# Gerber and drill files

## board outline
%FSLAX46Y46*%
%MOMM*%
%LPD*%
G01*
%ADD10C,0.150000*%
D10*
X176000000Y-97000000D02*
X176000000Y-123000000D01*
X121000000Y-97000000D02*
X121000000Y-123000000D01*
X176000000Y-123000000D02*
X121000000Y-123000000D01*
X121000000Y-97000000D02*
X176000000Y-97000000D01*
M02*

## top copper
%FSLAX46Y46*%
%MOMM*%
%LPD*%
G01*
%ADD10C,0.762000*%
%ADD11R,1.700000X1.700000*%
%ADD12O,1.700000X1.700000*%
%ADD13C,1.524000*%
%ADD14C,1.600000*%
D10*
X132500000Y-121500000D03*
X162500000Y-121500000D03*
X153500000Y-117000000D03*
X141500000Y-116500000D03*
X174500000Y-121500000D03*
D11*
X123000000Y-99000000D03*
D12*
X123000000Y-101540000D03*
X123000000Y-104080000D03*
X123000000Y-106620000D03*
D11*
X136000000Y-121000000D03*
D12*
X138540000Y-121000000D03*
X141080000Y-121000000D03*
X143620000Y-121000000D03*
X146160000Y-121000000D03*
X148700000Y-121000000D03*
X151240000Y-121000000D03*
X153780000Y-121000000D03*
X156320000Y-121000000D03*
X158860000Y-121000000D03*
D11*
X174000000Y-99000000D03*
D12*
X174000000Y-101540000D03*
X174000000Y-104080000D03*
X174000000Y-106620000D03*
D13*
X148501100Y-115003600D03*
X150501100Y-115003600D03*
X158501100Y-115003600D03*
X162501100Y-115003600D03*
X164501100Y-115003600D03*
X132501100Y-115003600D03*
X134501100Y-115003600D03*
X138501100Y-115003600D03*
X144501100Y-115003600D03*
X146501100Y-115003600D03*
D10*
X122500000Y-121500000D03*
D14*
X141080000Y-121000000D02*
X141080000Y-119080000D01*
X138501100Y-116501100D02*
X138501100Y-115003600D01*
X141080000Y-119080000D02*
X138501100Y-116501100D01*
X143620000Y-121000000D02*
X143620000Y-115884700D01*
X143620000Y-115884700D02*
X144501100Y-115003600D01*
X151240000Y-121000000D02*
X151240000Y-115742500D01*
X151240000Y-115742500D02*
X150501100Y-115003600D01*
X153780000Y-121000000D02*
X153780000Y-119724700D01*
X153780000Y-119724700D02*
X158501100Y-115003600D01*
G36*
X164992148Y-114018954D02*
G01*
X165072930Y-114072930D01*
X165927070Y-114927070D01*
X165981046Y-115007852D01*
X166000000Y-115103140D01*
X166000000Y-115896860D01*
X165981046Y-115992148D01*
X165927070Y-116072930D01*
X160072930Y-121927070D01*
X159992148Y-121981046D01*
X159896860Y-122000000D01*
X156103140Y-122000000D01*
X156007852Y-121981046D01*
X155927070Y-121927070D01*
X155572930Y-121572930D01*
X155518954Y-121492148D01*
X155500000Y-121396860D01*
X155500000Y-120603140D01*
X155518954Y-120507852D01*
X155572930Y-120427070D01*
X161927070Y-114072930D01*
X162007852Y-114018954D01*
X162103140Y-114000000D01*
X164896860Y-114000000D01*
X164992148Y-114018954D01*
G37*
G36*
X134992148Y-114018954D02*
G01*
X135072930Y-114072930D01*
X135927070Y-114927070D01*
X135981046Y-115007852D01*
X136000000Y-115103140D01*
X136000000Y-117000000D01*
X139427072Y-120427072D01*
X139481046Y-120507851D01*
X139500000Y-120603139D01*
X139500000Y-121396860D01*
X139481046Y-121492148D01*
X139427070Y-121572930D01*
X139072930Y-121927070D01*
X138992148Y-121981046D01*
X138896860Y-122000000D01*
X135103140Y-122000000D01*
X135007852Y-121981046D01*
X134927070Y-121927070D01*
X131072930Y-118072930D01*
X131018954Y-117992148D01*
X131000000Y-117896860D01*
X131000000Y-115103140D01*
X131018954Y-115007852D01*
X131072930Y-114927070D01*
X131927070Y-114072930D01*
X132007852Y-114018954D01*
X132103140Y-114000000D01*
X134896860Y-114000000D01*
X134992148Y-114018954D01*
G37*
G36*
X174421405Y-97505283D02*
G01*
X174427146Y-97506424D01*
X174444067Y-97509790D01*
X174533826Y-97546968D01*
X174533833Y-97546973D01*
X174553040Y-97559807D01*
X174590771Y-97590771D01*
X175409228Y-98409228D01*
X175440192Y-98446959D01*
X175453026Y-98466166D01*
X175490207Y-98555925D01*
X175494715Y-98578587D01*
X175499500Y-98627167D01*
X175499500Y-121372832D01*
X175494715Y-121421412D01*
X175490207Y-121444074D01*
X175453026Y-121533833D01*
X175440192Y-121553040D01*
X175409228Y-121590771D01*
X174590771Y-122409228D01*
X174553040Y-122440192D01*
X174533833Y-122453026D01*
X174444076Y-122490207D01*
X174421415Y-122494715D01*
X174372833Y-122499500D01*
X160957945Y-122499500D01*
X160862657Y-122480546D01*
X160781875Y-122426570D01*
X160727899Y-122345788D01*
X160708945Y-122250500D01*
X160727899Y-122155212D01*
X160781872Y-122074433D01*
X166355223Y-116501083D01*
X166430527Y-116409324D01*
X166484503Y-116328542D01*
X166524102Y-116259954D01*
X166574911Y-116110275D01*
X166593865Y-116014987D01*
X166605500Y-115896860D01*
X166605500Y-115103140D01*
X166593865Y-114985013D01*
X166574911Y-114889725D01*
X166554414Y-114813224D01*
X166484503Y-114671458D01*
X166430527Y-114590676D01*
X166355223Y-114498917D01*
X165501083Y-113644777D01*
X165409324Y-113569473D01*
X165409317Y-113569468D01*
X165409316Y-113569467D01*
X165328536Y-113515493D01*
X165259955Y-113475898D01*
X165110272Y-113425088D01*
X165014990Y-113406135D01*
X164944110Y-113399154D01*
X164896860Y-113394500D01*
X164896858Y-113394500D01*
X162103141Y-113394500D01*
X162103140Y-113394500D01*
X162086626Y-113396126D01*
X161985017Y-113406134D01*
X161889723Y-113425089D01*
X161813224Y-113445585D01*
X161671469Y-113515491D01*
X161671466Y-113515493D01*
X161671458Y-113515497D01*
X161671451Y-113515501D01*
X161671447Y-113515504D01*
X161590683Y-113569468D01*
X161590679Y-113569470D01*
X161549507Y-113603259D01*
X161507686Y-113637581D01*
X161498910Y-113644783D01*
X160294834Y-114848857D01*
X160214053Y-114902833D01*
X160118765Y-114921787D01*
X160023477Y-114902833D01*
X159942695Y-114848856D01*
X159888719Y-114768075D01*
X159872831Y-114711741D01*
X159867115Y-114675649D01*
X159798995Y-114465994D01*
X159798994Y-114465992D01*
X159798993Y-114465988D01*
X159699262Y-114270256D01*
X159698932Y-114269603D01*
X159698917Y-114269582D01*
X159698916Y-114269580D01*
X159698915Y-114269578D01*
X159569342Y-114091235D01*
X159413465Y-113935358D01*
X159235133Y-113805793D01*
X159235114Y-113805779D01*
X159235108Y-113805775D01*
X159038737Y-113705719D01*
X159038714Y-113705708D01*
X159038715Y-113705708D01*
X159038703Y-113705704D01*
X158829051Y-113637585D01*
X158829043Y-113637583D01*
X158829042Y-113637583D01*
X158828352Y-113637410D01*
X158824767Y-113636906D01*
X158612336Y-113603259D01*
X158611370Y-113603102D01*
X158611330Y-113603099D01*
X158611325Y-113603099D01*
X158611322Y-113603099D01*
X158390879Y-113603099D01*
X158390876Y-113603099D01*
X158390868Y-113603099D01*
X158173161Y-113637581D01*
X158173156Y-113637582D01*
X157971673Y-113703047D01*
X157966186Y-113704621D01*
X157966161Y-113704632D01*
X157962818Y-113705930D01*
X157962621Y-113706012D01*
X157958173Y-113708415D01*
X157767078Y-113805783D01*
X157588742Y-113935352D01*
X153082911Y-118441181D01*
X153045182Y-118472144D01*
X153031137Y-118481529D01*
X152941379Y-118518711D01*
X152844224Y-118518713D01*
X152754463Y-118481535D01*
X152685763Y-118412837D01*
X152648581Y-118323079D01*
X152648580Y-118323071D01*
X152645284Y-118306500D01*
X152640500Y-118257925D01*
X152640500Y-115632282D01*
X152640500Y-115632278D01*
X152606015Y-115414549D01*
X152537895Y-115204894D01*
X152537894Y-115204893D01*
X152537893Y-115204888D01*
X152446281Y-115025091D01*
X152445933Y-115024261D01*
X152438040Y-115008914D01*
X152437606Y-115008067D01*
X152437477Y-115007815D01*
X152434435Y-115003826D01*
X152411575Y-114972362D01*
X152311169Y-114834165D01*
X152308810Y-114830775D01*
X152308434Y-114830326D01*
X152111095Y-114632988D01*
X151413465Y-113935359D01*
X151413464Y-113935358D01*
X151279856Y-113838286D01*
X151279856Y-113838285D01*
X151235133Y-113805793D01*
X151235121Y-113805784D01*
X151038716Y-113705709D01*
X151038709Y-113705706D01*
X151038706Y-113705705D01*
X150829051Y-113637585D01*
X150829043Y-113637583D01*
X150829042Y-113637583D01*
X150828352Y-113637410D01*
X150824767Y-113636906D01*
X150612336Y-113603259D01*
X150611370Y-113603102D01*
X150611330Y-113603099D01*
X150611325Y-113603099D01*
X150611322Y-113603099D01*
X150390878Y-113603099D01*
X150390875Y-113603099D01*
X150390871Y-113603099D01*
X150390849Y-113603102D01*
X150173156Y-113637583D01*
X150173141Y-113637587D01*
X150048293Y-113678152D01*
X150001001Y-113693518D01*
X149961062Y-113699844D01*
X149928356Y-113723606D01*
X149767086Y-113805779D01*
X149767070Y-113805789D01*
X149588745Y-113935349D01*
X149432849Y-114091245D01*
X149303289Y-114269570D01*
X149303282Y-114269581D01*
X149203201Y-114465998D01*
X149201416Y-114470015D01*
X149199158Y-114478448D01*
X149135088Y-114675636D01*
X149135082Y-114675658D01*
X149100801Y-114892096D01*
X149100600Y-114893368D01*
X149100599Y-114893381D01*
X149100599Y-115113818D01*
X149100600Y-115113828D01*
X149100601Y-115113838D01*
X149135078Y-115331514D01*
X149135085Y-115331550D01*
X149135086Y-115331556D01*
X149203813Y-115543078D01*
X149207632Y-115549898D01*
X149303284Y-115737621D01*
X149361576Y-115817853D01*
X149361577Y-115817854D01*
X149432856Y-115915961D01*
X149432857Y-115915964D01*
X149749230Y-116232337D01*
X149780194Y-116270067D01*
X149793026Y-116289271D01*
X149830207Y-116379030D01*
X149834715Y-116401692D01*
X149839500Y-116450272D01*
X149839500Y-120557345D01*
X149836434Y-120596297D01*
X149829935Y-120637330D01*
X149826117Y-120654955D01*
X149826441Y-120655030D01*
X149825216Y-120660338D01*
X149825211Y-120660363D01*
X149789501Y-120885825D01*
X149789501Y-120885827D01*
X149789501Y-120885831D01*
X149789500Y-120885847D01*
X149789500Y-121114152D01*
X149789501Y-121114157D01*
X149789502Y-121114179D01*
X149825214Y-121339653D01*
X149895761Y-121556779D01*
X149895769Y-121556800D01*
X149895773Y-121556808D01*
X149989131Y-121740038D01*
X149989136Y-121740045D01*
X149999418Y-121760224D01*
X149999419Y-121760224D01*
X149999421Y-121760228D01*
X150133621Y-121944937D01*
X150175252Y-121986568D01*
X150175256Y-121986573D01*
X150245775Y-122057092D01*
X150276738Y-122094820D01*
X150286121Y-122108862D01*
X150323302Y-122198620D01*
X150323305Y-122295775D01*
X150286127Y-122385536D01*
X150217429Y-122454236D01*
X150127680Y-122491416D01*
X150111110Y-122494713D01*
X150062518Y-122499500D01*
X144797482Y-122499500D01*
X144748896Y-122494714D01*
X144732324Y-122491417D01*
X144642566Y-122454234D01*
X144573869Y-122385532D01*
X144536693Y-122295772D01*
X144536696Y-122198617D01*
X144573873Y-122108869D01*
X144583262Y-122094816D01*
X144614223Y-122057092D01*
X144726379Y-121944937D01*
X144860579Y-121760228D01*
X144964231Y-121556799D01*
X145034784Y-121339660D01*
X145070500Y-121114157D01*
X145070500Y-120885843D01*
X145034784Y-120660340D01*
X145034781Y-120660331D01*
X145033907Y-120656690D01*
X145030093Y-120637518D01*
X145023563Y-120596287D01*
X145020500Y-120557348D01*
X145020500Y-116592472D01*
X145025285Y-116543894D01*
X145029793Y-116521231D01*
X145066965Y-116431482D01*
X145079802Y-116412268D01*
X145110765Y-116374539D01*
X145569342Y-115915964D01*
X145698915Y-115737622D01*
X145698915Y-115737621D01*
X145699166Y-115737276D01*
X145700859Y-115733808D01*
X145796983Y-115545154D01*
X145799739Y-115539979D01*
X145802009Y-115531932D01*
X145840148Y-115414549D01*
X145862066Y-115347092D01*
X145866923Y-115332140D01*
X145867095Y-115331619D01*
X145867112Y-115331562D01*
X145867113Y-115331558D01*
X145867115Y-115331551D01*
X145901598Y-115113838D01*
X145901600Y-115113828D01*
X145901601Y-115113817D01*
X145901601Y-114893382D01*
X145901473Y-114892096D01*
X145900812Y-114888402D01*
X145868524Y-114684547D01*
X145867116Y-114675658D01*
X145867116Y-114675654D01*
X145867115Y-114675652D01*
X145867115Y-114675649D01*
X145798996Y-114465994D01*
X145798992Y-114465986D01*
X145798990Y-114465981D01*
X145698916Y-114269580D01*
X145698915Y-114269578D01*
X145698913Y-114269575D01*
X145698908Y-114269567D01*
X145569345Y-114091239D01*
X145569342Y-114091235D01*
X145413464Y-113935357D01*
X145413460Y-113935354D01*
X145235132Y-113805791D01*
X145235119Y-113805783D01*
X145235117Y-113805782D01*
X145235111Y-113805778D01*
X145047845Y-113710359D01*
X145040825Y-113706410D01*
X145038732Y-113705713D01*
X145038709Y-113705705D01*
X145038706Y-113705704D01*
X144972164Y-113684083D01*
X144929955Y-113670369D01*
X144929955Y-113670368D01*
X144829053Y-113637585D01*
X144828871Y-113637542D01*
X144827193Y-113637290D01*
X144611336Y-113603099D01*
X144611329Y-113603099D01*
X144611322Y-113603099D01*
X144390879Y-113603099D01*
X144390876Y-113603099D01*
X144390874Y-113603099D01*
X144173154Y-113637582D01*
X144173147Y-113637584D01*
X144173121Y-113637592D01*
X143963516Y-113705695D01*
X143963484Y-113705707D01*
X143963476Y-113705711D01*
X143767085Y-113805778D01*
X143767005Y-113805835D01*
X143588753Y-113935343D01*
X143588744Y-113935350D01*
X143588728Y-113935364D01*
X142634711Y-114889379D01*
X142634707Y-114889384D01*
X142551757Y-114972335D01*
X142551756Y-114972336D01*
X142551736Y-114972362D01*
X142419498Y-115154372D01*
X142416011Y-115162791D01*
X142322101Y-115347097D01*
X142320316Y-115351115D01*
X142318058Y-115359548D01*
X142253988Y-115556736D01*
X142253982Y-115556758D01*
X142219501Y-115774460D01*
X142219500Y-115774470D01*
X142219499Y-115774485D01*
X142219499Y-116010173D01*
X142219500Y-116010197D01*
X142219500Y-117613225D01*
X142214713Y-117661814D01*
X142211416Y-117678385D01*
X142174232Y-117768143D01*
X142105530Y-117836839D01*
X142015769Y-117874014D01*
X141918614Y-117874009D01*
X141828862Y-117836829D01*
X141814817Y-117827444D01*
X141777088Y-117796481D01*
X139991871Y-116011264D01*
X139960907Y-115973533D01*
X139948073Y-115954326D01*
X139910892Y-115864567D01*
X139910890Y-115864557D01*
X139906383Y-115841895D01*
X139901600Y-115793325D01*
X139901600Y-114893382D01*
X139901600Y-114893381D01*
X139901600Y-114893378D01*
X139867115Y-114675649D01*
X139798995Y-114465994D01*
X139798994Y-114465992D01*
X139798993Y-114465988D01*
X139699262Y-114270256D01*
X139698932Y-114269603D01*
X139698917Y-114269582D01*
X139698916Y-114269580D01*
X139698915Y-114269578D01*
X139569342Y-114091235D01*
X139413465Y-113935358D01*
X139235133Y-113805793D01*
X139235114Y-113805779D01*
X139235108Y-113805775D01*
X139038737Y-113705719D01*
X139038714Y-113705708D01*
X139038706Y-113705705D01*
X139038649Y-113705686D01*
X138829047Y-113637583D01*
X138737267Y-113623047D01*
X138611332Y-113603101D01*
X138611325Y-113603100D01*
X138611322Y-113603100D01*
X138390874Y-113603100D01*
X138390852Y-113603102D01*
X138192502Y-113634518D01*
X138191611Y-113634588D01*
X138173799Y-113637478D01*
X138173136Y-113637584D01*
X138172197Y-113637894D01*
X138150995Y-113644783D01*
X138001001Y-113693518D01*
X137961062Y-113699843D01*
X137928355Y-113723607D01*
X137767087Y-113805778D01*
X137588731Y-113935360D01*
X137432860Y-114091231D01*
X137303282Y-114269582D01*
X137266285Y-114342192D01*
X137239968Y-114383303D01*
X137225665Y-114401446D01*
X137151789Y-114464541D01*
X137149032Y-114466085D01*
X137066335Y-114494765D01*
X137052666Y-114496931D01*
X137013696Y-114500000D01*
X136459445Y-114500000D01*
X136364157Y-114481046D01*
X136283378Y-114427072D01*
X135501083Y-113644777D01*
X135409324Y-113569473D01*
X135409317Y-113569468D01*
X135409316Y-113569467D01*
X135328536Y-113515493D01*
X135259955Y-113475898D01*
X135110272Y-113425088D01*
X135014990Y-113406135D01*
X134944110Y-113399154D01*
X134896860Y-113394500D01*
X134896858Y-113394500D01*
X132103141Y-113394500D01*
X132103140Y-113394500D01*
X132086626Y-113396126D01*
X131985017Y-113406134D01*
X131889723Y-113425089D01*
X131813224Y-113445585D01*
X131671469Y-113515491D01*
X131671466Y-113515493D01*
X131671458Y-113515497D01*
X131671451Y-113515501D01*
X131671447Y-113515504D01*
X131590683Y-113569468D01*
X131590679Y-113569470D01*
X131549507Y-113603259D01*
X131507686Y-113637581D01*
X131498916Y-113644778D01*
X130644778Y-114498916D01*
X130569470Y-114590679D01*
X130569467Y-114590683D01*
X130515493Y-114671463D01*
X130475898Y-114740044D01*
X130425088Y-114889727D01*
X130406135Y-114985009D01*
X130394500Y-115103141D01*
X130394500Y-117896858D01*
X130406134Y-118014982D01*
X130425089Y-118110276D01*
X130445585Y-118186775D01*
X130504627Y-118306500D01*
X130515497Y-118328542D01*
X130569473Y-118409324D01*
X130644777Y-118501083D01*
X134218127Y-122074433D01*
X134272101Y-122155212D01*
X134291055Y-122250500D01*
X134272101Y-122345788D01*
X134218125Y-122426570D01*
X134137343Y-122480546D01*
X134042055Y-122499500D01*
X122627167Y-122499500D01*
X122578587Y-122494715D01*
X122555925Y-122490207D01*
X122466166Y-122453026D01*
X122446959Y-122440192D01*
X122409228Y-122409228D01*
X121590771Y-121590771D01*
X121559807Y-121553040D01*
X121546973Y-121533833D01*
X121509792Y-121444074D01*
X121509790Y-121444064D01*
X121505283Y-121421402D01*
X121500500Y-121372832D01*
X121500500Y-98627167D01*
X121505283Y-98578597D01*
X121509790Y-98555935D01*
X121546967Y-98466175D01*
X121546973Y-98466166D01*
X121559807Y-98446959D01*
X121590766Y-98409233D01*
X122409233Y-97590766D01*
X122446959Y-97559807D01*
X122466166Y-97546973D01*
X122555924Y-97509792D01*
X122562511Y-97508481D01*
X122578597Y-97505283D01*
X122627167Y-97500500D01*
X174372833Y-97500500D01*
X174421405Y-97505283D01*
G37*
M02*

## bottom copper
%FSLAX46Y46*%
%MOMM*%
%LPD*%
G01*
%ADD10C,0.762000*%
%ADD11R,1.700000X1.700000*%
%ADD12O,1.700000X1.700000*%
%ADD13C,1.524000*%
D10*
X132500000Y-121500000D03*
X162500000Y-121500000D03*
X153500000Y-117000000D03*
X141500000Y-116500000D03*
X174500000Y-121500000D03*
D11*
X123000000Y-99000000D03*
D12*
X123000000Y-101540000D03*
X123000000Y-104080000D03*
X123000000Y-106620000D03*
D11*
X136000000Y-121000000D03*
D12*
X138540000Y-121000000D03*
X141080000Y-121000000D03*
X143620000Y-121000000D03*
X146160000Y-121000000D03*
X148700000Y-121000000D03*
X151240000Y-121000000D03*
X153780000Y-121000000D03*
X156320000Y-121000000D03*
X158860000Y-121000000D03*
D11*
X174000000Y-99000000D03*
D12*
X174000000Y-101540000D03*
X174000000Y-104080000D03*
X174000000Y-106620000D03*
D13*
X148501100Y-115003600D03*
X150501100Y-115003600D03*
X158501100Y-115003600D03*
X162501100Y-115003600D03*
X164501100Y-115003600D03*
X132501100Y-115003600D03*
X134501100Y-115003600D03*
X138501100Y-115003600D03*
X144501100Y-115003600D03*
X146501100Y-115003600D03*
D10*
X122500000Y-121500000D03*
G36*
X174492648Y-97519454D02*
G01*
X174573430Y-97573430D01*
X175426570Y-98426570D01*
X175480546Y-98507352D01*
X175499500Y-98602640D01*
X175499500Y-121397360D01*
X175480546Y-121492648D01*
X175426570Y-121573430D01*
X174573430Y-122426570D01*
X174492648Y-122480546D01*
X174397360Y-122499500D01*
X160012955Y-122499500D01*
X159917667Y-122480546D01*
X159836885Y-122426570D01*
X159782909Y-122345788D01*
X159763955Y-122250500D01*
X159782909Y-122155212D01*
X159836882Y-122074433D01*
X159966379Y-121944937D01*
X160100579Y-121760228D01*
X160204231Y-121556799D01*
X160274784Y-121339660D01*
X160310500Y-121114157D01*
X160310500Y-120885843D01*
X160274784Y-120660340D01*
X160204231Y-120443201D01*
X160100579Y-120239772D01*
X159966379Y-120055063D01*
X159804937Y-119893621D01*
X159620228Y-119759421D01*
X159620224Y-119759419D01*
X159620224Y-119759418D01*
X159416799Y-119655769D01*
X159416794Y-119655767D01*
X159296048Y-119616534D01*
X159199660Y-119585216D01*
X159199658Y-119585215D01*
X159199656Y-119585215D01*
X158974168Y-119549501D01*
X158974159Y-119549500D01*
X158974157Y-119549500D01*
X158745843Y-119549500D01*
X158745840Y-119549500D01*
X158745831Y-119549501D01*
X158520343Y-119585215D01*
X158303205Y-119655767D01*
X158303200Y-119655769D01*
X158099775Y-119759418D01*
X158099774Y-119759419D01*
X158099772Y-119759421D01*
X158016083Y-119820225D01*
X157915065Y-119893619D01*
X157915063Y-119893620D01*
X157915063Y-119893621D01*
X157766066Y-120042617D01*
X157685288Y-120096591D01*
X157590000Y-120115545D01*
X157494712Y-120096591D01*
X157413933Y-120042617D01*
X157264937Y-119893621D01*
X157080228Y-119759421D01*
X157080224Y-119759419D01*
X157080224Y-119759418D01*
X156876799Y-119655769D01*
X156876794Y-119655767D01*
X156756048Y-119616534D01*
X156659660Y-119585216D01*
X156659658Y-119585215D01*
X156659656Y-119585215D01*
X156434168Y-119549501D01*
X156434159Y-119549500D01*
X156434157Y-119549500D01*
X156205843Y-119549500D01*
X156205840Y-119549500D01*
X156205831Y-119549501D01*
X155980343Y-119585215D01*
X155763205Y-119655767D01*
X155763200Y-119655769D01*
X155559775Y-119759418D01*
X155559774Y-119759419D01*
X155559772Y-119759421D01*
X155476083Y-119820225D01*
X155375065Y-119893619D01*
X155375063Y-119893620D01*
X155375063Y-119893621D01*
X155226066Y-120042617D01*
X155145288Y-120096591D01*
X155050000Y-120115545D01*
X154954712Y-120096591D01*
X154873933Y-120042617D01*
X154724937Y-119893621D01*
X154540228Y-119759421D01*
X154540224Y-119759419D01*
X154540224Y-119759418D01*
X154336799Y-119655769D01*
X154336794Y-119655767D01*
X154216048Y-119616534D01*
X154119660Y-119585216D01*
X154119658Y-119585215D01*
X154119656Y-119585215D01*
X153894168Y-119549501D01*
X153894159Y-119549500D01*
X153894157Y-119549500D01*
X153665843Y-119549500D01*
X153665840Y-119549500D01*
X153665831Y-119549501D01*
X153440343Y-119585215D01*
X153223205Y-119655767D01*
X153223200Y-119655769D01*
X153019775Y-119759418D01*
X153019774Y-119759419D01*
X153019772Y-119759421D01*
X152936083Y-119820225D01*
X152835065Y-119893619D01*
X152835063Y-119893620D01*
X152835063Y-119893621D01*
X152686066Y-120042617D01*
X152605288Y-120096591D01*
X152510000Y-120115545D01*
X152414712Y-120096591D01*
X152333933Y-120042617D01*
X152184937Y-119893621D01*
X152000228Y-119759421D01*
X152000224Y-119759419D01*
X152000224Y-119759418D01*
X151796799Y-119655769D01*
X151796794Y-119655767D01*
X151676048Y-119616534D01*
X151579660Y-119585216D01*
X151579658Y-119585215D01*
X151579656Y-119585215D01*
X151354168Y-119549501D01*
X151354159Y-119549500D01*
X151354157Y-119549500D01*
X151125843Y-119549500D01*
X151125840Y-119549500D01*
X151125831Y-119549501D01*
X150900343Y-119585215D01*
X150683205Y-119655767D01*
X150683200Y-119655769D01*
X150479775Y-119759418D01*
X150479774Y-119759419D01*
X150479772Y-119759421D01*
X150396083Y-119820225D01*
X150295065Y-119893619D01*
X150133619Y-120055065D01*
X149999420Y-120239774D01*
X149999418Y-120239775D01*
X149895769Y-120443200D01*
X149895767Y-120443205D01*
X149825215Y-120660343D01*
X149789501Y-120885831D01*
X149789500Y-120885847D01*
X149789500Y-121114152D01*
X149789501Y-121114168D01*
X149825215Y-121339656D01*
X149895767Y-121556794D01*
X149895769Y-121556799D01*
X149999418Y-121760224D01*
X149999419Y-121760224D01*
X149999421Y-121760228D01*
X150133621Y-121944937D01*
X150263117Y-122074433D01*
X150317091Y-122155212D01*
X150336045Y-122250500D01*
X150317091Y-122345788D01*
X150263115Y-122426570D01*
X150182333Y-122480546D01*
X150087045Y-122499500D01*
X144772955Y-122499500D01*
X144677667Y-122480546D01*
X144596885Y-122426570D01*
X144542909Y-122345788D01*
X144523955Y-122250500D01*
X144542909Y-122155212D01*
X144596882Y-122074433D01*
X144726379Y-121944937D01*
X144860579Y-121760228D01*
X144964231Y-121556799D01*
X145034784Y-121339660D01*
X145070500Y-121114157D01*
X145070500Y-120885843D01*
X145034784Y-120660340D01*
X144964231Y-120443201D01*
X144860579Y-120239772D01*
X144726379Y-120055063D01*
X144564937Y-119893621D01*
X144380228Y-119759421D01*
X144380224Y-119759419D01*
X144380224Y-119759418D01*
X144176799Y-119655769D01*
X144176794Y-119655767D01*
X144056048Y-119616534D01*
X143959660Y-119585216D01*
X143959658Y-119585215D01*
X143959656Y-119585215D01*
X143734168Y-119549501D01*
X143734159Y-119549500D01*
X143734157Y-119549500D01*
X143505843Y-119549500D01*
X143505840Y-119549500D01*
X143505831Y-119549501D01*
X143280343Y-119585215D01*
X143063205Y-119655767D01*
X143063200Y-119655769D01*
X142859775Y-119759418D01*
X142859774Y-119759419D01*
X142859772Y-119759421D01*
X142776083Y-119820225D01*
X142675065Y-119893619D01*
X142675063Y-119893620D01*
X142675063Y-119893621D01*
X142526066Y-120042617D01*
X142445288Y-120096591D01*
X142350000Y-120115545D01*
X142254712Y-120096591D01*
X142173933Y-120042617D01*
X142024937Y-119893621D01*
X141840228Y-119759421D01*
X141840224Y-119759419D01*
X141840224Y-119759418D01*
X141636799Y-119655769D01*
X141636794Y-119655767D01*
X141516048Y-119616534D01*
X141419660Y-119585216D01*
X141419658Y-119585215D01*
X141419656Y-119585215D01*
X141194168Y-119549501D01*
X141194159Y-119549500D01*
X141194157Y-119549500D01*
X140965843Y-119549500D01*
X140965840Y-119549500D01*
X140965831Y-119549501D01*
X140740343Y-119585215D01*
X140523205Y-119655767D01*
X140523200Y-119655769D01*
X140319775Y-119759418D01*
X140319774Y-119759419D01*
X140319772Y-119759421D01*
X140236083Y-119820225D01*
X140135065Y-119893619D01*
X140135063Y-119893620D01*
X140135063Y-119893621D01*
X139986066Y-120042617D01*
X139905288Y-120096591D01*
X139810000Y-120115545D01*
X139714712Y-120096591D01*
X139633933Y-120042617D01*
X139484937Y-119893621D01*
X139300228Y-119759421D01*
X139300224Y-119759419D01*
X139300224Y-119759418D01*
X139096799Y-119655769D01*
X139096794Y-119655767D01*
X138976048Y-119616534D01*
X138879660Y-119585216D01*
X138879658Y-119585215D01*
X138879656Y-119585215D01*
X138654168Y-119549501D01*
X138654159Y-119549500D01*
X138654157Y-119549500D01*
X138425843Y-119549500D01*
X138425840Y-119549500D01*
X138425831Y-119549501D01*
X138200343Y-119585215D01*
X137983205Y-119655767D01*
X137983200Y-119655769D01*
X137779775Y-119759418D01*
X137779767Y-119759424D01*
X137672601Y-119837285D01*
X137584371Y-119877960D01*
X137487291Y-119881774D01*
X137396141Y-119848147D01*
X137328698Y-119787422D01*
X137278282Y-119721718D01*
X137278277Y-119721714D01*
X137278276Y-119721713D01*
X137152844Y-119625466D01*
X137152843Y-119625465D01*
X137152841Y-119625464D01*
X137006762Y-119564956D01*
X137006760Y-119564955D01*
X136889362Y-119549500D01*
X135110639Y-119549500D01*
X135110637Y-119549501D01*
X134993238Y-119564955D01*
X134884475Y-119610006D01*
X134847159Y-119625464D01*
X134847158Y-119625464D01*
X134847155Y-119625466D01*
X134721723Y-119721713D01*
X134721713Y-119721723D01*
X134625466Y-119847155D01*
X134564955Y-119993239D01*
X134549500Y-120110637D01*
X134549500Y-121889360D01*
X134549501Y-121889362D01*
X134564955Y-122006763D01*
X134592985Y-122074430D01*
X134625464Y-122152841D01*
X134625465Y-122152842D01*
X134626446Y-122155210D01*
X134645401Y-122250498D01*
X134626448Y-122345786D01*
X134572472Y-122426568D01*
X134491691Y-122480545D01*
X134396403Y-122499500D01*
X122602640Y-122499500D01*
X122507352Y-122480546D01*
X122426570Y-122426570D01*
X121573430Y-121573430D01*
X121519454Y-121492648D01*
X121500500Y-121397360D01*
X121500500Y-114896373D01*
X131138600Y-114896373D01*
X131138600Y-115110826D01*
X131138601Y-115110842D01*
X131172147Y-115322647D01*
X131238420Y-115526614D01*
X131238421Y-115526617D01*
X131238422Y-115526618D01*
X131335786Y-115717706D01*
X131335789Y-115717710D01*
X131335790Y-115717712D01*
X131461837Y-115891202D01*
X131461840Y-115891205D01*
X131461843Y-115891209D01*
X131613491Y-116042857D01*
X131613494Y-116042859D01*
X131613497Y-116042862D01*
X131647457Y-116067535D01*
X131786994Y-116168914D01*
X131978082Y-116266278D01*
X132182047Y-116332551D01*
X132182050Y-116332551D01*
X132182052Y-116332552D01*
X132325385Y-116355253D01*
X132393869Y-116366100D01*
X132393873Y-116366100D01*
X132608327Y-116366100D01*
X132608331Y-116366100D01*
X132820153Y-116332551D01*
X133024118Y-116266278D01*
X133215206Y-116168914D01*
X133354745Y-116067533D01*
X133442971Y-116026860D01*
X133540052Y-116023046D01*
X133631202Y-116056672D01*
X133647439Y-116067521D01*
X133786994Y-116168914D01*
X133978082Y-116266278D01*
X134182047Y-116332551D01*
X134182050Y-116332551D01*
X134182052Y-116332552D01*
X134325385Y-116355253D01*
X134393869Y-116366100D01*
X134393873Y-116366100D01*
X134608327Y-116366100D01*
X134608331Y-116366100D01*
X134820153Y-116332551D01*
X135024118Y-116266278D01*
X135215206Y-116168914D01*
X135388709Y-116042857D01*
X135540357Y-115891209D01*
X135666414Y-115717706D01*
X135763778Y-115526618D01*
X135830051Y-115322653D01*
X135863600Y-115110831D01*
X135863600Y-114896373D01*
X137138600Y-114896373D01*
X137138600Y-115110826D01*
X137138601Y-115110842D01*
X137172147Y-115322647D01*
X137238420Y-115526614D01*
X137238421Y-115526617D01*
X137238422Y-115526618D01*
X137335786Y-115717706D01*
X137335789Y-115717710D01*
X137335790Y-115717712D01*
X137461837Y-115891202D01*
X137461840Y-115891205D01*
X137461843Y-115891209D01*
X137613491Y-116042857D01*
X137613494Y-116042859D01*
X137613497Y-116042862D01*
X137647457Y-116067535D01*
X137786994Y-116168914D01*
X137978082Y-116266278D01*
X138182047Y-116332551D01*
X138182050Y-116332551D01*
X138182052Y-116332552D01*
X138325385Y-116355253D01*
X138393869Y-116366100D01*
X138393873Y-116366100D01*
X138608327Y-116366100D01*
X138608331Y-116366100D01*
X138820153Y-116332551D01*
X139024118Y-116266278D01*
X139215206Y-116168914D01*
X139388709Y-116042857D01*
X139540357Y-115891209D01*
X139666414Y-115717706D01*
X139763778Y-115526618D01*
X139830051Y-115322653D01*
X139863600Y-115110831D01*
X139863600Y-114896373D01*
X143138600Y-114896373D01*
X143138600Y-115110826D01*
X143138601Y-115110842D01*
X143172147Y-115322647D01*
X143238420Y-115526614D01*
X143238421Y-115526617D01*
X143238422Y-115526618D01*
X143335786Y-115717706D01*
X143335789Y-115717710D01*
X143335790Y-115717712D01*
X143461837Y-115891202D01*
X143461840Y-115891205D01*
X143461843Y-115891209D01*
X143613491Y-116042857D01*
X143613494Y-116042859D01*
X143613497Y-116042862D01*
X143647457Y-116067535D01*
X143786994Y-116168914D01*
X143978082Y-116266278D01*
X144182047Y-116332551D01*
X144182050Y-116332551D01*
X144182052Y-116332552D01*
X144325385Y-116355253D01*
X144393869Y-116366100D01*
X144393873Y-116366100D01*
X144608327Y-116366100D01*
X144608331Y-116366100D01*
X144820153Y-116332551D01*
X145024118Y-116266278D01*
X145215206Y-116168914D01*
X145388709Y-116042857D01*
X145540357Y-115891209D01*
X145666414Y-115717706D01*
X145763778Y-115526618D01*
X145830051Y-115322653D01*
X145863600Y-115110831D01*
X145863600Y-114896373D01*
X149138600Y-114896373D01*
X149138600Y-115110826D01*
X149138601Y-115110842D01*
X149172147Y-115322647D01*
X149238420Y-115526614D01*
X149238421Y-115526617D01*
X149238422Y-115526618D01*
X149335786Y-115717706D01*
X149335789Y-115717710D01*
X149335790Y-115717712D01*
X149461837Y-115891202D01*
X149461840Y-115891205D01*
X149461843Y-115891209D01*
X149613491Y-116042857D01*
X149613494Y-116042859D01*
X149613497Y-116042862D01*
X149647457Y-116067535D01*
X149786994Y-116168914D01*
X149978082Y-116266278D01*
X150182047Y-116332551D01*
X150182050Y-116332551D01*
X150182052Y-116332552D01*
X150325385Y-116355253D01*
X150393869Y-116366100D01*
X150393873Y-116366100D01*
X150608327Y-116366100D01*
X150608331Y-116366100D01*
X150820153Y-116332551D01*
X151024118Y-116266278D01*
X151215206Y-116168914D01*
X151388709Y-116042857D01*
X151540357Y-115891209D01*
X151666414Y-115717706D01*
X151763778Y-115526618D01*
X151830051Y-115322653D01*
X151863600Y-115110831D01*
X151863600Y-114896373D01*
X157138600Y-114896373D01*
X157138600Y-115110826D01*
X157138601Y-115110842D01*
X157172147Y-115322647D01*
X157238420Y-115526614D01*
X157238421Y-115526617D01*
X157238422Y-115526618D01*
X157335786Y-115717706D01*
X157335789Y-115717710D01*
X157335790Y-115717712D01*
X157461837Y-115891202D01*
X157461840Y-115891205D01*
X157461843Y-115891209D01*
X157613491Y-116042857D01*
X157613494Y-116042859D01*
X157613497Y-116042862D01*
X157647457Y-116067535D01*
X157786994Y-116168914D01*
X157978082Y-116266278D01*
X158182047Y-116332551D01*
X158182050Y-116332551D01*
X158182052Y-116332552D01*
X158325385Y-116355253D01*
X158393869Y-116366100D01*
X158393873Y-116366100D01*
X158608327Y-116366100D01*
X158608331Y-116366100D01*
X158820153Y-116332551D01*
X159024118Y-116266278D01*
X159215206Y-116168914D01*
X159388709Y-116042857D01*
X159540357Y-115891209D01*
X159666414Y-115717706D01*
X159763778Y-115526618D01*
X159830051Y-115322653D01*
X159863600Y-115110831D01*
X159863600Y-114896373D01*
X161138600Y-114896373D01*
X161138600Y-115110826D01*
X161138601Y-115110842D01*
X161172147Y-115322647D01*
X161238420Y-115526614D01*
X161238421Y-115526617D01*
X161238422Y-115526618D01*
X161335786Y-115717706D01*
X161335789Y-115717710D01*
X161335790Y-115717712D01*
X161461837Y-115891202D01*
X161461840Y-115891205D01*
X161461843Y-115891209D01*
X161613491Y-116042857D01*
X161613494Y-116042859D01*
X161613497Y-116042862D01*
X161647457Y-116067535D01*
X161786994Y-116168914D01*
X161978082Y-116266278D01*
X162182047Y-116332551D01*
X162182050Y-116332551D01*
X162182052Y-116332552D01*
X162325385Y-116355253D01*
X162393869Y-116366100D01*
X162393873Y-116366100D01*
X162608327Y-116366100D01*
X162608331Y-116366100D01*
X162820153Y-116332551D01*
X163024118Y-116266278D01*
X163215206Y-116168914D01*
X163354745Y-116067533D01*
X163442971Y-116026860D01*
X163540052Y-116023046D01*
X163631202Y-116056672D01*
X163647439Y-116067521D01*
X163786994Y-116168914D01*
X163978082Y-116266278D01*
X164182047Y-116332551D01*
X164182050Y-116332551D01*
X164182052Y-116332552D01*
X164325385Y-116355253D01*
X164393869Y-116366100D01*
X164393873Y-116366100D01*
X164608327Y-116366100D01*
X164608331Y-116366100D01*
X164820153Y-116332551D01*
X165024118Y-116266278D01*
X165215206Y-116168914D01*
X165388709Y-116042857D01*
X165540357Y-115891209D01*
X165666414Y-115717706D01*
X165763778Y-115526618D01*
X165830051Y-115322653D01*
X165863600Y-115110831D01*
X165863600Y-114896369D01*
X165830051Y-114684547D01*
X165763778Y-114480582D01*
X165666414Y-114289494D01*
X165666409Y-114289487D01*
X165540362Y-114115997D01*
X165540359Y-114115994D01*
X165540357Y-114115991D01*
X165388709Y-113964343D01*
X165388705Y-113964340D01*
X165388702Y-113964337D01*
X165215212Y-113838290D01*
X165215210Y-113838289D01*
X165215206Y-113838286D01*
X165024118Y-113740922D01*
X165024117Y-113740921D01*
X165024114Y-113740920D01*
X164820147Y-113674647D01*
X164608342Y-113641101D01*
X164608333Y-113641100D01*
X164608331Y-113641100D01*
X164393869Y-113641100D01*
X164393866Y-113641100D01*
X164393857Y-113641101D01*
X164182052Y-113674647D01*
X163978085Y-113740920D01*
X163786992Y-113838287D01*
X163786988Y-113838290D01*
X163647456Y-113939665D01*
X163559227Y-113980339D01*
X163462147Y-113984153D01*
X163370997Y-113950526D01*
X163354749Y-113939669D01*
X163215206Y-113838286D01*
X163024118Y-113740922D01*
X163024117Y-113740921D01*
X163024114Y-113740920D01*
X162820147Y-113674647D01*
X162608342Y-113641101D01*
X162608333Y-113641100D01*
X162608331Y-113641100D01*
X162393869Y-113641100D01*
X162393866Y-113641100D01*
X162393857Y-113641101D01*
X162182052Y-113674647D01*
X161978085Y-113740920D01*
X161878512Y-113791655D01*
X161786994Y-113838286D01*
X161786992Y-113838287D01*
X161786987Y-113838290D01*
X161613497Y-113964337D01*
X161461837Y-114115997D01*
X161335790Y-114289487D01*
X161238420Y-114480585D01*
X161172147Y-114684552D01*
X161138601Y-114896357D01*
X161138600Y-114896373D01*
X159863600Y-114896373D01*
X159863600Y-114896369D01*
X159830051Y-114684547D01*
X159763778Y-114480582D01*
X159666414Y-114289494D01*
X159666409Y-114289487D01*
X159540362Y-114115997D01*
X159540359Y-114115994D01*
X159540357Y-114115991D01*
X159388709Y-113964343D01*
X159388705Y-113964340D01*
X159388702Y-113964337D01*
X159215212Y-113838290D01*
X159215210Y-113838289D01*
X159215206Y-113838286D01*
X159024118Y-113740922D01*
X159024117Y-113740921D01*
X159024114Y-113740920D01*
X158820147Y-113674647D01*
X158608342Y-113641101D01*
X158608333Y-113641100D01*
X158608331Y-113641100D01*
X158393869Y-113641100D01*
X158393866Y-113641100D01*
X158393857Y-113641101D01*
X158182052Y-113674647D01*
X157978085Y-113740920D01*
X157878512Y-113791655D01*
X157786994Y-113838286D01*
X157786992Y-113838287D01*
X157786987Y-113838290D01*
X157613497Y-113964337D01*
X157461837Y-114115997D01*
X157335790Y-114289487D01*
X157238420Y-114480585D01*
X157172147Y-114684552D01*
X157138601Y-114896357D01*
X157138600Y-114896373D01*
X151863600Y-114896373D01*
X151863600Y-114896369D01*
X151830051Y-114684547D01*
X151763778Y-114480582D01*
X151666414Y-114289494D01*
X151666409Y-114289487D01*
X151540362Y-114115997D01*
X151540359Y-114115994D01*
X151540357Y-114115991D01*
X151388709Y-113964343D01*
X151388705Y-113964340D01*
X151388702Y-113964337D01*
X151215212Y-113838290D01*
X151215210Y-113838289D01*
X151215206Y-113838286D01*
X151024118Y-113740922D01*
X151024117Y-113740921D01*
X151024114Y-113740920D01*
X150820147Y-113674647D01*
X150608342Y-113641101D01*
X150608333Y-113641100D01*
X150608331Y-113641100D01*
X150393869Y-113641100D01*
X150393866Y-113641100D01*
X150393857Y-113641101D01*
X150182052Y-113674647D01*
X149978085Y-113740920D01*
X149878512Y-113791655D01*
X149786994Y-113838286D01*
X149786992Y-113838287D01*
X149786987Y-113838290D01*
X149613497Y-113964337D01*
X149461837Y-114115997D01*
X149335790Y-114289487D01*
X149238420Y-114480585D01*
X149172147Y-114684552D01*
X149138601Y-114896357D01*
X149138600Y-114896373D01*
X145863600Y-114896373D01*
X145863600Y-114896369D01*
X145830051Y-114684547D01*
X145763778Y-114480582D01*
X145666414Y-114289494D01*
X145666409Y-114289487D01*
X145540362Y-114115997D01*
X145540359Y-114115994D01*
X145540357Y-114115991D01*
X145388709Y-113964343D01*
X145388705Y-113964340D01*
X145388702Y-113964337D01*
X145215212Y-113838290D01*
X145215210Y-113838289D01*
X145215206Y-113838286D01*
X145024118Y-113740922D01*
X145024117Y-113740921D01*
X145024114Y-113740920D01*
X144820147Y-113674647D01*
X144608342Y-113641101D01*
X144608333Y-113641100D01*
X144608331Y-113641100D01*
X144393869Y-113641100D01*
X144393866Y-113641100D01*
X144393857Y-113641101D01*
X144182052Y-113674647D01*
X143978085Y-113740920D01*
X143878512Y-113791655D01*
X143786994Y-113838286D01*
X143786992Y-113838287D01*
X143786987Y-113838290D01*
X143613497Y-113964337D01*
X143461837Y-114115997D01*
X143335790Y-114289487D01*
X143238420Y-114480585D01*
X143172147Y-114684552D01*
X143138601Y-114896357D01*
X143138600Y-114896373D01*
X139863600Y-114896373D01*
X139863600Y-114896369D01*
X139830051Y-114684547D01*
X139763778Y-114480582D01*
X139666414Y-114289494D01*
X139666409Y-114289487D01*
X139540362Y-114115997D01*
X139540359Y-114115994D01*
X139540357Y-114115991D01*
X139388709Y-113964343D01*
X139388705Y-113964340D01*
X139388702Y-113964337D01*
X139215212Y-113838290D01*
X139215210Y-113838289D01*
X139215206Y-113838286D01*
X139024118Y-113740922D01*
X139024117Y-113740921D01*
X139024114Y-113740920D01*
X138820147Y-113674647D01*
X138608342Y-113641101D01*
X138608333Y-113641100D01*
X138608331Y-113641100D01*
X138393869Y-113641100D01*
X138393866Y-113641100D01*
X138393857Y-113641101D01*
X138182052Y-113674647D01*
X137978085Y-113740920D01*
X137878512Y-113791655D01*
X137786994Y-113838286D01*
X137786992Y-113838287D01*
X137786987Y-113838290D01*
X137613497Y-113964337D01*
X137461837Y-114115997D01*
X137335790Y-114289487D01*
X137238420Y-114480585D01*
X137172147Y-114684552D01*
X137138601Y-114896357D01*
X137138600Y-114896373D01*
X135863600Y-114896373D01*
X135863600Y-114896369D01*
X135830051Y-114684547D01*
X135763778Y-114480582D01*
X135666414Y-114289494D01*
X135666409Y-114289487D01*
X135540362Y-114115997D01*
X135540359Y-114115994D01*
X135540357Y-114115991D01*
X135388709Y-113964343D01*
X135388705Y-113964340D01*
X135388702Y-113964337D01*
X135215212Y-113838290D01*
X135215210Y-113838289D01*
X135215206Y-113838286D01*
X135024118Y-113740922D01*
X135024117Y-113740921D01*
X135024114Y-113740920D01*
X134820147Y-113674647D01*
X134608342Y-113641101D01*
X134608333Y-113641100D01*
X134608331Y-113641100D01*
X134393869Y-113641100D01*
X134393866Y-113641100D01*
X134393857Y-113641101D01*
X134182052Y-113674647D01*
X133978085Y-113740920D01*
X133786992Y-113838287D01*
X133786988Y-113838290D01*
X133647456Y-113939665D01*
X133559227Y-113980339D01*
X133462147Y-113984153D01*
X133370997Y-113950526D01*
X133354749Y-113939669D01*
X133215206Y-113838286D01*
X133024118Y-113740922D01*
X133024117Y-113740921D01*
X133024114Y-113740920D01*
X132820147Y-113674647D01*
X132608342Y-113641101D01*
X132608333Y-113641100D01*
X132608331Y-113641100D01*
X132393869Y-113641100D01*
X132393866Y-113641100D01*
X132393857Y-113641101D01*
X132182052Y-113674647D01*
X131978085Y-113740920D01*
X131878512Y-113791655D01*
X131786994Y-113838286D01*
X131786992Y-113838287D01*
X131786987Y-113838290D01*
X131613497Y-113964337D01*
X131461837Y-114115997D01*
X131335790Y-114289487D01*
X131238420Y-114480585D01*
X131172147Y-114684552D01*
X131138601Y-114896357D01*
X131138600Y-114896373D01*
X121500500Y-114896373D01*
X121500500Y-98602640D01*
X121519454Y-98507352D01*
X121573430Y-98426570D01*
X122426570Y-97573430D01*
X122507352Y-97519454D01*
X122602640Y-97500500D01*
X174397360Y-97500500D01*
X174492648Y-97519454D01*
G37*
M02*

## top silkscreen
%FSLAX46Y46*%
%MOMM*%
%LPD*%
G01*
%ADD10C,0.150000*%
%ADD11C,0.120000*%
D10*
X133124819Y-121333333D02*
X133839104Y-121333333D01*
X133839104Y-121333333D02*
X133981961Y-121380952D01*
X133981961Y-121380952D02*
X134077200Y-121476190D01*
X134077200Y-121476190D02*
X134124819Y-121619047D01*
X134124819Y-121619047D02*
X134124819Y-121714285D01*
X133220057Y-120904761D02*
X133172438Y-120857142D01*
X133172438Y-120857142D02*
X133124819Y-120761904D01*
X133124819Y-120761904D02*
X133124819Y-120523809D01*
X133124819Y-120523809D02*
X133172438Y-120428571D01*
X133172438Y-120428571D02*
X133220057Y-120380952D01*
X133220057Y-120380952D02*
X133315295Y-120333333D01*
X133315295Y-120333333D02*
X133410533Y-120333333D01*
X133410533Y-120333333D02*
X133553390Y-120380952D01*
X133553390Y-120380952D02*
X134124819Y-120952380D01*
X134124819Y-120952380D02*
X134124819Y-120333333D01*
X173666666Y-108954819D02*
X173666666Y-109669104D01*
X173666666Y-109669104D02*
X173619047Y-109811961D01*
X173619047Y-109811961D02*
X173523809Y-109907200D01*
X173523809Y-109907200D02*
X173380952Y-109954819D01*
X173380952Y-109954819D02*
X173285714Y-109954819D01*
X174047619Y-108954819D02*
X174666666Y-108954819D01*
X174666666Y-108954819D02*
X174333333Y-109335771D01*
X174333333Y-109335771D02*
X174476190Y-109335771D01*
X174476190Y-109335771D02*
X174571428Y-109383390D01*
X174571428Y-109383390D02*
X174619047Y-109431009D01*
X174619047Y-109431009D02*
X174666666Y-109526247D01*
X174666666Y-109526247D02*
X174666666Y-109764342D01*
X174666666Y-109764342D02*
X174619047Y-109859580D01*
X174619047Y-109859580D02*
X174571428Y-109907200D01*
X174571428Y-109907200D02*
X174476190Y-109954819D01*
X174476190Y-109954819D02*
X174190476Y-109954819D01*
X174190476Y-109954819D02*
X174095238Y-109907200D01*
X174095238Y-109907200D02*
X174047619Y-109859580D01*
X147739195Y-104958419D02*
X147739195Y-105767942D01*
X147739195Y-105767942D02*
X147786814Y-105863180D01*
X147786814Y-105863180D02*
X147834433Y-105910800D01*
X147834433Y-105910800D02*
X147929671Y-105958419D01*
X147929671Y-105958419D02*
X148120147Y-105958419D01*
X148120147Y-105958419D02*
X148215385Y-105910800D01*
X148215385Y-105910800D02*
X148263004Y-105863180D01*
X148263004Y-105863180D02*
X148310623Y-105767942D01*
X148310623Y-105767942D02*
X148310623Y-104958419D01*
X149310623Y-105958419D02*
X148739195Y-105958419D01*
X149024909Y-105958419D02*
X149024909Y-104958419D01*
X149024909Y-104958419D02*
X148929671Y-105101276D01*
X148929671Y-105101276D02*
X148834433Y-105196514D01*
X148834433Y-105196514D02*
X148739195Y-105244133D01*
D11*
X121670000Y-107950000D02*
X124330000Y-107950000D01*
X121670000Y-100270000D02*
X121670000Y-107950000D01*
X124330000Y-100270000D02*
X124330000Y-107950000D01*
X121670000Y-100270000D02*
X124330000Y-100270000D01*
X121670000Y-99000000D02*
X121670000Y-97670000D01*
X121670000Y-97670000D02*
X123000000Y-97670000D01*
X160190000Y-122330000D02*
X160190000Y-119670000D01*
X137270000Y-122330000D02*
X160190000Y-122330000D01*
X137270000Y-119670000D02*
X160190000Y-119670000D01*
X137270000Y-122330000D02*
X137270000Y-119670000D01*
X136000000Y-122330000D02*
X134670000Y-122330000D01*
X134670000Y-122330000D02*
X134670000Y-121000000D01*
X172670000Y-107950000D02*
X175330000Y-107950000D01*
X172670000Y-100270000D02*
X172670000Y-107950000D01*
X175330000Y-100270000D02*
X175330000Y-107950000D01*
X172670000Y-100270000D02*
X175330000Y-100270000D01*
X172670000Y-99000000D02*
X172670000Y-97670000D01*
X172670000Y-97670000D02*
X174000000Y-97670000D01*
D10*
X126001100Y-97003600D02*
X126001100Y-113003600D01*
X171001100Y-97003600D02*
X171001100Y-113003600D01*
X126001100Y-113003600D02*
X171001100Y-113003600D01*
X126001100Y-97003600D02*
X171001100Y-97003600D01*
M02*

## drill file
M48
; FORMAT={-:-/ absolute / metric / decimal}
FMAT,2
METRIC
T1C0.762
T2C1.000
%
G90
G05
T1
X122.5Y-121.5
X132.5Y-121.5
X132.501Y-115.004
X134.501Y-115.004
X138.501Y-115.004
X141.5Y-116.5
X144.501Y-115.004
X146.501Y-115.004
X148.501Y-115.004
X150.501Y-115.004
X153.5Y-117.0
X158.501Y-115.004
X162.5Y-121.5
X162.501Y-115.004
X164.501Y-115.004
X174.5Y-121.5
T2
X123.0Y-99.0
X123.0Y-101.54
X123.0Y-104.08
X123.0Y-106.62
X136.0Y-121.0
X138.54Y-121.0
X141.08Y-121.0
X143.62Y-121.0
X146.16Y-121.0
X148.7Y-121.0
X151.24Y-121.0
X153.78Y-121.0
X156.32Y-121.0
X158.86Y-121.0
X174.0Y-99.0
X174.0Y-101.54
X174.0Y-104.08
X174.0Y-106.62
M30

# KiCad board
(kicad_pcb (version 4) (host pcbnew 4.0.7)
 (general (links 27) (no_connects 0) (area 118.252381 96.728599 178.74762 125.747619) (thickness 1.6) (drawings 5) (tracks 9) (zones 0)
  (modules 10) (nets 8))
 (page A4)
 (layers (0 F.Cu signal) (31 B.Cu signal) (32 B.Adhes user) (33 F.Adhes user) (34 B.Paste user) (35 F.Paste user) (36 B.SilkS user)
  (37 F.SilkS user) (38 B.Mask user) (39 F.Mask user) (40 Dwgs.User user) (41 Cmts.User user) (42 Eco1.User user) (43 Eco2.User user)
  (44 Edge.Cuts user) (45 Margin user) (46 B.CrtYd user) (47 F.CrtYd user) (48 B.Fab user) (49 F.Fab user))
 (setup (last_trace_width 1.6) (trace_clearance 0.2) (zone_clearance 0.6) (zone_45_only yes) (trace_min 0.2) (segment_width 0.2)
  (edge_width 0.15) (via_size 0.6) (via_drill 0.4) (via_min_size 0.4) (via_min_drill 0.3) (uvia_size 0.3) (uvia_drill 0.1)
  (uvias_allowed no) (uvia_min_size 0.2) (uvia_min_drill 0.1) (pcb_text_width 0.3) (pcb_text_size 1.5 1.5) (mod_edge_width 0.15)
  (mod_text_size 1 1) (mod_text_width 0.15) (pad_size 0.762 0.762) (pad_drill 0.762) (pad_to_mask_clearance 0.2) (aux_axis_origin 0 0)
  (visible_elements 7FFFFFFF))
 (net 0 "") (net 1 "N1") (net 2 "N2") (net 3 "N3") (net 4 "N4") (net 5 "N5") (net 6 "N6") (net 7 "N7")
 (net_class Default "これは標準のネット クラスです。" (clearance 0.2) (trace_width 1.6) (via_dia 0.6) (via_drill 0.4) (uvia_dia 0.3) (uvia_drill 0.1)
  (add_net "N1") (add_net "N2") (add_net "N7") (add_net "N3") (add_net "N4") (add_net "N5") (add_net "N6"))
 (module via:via (layer F.Cu) (at 132.5 121.5)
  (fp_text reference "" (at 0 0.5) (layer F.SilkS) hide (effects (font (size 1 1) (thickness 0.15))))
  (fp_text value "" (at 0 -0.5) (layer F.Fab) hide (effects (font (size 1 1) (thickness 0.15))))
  (pad 1 thru_hole circle (at 0 0) (size 0.762 0.762) (drill 0.762) (layers *.Cu *.Mask) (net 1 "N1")))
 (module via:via (layer F.Cu) (at 162.5 121.5)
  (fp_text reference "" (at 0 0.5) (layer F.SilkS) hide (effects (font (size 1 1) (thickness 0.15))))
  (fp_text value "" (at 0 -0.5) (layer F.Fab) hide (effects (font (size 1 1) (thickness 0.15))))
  (pad 1 thru_hole circle (at 0 0) (size 0.762 0.762) (drill 0.762) (layers *.Cu *.Mask) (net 1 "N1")))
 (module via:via (layer F.Cu) (at 153.5 117)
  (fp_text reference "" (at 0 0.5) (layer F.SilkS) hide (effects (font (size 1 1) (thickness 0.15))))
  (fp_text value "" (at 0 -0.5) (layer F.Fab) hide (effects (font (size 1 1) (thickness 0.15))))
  (pad 1 thru_hole circle (at 0 0) (size 0.762 0.762) (drill 0.762) (layers *.Cu *.Mask) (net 1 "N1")))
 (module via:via (layer F.Cu) (at 141.5 116.5)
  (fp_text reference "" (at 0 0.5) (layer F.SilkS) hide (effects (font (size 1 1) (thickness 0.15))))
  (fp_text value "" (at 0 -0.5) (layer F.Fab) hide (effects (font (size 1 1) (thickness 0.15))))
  (pad 1 thru_hole circle (at 0 0) (size 0.762 0.762) (drill 0.762) (layers *.Cu *.Mask) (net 1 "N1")))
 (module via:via (layer F.Cu) (at 174.5 121.5)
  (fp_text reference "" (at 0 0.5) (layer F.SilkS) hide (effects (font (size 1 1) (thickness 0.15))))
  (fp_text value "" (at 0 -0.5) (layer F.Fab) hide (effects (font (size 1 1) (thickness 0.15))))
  (pad 1 thru_hole circle (at 0 0) (size 0.762 0.762) (drill 0.762) (layers *.Cu *.Mask) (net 1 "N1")))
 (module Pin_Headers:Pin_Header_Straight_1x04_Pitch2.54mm (layer F.Cu) (at 123 99)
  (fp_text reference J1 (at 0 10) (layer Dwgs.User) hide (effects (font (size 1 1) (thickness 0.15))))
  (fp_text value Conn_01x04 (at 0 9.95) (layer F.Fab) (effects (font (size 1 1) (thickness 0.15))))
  (fp_line (start -1.33 8.95) (end 1.33 8.95) (layer F.SilkS) (width 0.12))
  (fp_line (start -1.33 1.27) (end -1.33 8.95) (layer F.SilkS) (width 0.12))
  (fp_line (start 1.33 1.27) (end 1.33 8.95) (layer F.SilkS) (width 0.12))
  (fp_line (start -1.33 1.27) (end 1.33 1.27) (layer F.SilkS) (width 0.12))
  (fp_line (start -1.33 0) (end -1.33 -1.33) (layer F.SilkS) (width 0.12))
  (fp_line (start -1.33 -1.33) (end 0 -1.33) (layer F.SilkS) (width 0.12))
  (pad 1 thru_hole rect (at 0 0) (size 1.7 1.7) (drill 1) (layers *.Cu *.Mask) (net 1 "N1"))
  (pad 2 thru_hole oval (at 0 2.54) (size 1.7 1.7) (drill 1) (layers *.Cu *.Mask) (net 1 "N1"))
  (pad 3 thru_hole oval (at 0 5.08) (size 1.7 1.7) (drill 1) (layers *.Cu *.Mask) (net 1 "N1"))
  (pad 4 thru_hole oval (at 0 7.62) (size 1.7 1.7) (drill 1) (layers *.Cu *.Mask) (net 1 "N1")))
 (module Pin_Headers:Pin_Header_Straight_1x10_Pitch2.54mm (layer F.Cu) (at 136 121 90)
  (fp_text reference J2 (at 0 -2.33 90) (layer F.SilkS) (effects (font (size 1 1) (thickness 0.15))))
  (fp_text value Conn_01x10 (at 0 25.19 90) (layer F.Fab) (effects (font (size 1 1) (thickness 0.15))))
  (fp_line (start -1.33 24.19) (end 1.33 24.19) (layer F.SilkS) (width 0.12))
  (fp_line (start -1.33 1.27) (end -1.33 24.19) (layer F.SilkS) (width 0.12))
  (fp_line (start 1.33 1.27) (end 1.33 24.19) (layer F.SilkS) (width 0.12))
  (fp_line (start -1.33 1.27) (end 1.33 1.27) (layer F.SilkS) (width 0.12))
  (fp_line (start -1.33 0) (end -1.33 -1.33) (layer F.SilkS) (width 0.12))
  (fp_line (start -1.33 -1.33) (end 0 -1.33) (layer F.SilkS) (width 0.12))
  (pad 1 thru_hole rect (at 0 0 90) (size 1.7 1.7) (drill 1) (layers *.Cu *.Mask) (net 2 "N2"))
  (pad 2 thru_hole oval (at 0 2.54 90) (size 1.7 1.7) (drill 1) (layers *.Cu *.Mask) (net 2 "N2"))
  (pad 3 thru_hole oval (at 0 5.08 90) (size 1.7 1.7) (drill 1) (layers *.Cu *.Mask) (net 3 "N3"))
  (pad 4 thru_hole oval (at 0 7.62 90) (size 1.7 1.7) (drill 1) (layers *.Cu *.Mask) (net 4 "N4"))
  (pad 5 thru_hole oval (at 0 10.16 90) (size 1.7 1.7) (drill 1) (layers *.Cu *.Mask) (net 1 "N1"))
  (pad 6 thru_hole oval (at 0 12.7 90) (size 1.7 1.7) (drill 1) (layers *.Cu *.Mask) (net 1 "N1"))
  (pad 7 thru_hole oval (at 0 15.24 90) (size 1.7 1.7) (drill 1) (layers *.Cu *.Mask) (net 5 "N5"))
  (pad 8 thru_hole oval (at 0 17.78 90) (size 1.7 1.7) (drill 1) (layers *.Cu *.Mask) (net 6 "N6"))
  (pad 9 thru_hole oval (at 0 20.32 90) (size 1.7 1.7) (drill 1) (layers *.Cu *.Mask) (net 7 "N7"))
  (pad 10 thru_hole oval (at 0 22.86 90) (size 1.7 1.7) (drill 1) (layers *.Cu *.Mask) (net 7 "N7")))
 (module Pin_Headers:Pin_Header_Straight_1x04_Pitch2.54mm (layer F.Cu) (at 174 99)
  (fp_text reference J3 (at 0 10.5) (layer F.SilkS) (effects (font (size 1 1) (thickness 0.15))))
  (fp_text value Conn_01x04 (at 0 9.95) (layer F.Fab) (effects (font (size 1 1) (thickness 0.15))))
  (fp_line (start -1.33 8.95) (end 1.33 8.95) (layer F.SilkS) (width 0.12))
  (fp_line (start -1.33 1.27) (end -1.33 8.95) (layer F.SilkS) (width 0.12))
  (fp_line (start 1.33 1.27) (end 1.33 8.95) (layer F.SilkS) (width 0.12))
  (fp_line (start -1.33 1.27) (end 1.33 1.27) (layer F.SilkS) (width 0.12))
  (fp_line (start -1.33 0) (end -1.33 -1.33) (layer F.SilkS) (width 0.12))
  (fp_line (start -1.33 -1.33) (end 0 -1.33) (layer F.SilkS) (width 0.12))
  (pad 1 thru_hole rect (at 0 0) (size 1.7 1.7) (drill 1) (layers *.Cu *.Mask) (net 1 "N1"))
  (pad 2 thru_hole oval (at 0 2.54) (size 1.7 1.7) (drill 1) (layers *.Cu *.Mask) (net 1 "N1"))
  (pad 3 thru_hole oval (at 0 5.08) (size 1.7 1.7) (drill 1) (layers *.Cu *.Mask) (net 1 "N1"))
  (pad 4 thru_hole oval (at 0 7.62) (size 1.7 1.7) (drill 1) (layers *.Cu *.Mask) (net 1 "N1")))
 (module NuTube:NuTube (layer F.Cu) (at 148.5011 105.0036)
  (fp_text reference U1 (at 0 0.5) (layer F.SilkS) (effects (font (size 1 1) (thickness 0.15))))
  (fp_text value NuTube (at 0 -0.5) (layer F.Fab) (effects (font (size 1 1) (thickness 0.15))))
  (fp_line (start -22.5 -8) (end -22.5 8) (layer F.SilkS) (width 0.15))
  (fp_line (start 22.5 -8) (end 22.5 8) (layer F.SilkS) (width 0.15))
  (fp_line (start -22.5 8) (end 22.5 8) (layer F.SilkS) (width 0.15))
  (fp_line (start -22.5 -8) (end 22.5 -8) (layer F.SilkS) (width 0.15))
  (pad 6 thru_hole circle (at 0 10) (size 1.524 1.524) (drill 0.762) (layers *.Cu *.Mask) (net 1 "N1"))
  (pad 7 thru_hole circle (at 2 10) (size 1.524 1.524) (drill 0.762) (layers *.Cu *.Mask) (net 5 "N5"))
  (pad 8 thru_hole circle (at 10 10) (size 1.524 1.524) (drill 0.762) (layers *.Cu *.Mask) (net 6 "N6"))
  (pad 9 thru_hole circle (at 14 10) (size 1.524 1.524) (drill 0.762) (layers *.Cu *.Mask) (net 7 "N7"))
  (pad 10 thru_hole circle (at 16 10) (size 1.524 1.524) (drill 0.762) (layers *.Cu *.Mask) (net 7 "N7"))
  (pad 1 thru_hole circle (at -16 10) (size 1.524 1.524) (drill 0.762) (layers *.Cu *.Mask) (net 2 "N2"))
  (pad 2 thru_hole circle (at -14 10) (size 1.524 1.524) (drill 0.762) (layers *.Cu *.Mask) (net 2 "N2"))
  (pad 3 thru_hole circle (at -10 10) (size 1.524 1.524) (drill 0.762) (layers *.Cu *.Mask) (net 3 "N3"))
  (pad 4 thru_hole circle (at -4 10) (size 1.524 1.524) (drill 0.762) (layers *.Cu *.Mask) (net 4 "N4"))
  (pad 5 thru_hole circle (at -2 10) (size 1.524 1.524) (drill 0.762) (layers *.Cu *.Mask) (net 1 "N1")))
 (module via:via (layer F.Cu) (at 122.5 121.5)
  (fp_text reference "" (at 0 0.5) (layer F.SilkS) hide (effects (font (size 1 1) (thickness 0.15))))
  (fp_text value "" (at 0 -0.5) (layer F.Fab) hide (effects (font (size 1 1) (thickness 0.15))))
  (pad 1 thru_hole circle (at 0 0) (size 0.762 0.762) (drill 0.762) (layers *.Cu *.Mask) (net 1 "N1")))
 (gr_line (start 176 97) (end 176 123) (angle 90) (layer Edge.Cuts) (width 0.15))
 (gr_line (start 121 97) (end 121 123) (angle 90) (layer Edge.Cuts) (width 0.15))
 (gr_line (start 176 123) (end 121 123) (angle 90) (layer Edge.Cuts) (width 0.15))
 (gr_line (start 121 97) (end 176 97) (angle 90) (layer Edge.Cuts) (width 0.15))
 (segment (start 141.08 121) (end 141.08 119.08) (width 1.6) (layer F.Cu) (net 3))
 (segment (start 138.5011 116.5011) (end 138.5011 115.0036) (width 1.6) (layer F.Cu) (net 3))
 (segment (start 141.08 119.08) (end 138.5011 116.5011) (width 1.6) (layer F.Cu) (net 3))
 (segment (start 143.62 121) (end 143.62 115.8847) (width 1.6) (layer F.Cu) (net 4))
 (segment (start 143.62 115.8847) (end 144.5011 115.0036) (width 1.6) (layer F.Cu) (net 4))
 (segment (start 151.24 121) (end 151.24 115.7425) (width 1.6) (layer F.Cu) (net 5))
 (segment (start 151.24 115.7425) (end 150.5011 115.0036) (width 1.6) (layer F.Cu) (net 5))
 (segment (start 153.78 121) (end 153.78 119.7247) (width 1.6) (layer F.Cu) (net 6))
 (segment (start 153.78 119.7247) (end 158.5011 115.0036) (width 1.6) (layer F.Cu) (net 6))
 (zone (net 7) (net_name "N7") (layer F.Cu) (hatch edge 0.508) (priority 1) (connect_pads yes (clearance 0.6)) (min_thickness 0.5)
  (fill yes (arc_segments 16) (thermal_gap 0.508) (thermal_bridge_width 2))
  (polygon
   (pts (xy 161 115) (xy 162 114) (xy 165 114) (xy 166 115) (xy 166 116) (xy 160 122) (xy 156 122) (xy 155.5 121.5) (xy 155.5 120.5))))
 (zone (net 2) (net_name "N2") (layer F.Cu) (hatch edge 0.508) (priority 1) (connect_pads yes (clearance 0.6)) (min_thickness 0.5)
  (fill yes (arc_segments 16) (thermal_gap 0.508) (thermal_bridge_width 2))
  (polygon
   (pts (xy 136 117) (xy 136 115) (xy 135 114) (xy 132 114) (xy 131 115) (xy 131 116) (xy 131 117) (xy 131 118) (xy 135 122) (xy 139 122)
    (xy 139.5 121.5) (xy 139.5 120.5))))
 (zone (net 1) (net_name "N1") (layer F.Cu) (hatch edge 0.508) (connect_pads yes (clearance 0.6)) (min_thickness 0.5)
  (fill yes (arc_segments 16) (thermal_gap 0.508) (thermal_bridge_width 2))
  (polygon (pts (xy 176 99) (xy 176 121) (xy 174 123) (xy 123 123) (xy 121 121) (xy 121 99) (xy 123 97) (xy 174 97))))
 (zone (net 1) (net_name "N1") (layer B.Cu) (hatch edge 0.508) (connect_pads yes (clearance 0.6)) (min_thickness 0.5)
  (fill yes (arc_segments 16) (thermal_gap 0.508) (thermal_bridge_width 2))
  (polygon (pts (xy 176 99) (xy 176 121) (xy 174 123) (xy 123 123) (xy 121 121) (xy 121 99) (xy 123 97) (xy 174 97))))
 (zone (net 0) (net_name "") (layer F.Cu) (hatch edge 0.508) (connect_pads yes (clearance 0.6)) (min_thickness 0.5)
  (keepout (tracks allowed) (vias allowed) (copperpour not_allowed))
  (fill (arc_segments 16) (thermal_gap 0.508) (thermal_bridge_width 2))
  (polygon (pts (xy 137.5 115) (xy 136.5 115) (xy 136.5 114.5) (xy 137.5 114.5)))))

